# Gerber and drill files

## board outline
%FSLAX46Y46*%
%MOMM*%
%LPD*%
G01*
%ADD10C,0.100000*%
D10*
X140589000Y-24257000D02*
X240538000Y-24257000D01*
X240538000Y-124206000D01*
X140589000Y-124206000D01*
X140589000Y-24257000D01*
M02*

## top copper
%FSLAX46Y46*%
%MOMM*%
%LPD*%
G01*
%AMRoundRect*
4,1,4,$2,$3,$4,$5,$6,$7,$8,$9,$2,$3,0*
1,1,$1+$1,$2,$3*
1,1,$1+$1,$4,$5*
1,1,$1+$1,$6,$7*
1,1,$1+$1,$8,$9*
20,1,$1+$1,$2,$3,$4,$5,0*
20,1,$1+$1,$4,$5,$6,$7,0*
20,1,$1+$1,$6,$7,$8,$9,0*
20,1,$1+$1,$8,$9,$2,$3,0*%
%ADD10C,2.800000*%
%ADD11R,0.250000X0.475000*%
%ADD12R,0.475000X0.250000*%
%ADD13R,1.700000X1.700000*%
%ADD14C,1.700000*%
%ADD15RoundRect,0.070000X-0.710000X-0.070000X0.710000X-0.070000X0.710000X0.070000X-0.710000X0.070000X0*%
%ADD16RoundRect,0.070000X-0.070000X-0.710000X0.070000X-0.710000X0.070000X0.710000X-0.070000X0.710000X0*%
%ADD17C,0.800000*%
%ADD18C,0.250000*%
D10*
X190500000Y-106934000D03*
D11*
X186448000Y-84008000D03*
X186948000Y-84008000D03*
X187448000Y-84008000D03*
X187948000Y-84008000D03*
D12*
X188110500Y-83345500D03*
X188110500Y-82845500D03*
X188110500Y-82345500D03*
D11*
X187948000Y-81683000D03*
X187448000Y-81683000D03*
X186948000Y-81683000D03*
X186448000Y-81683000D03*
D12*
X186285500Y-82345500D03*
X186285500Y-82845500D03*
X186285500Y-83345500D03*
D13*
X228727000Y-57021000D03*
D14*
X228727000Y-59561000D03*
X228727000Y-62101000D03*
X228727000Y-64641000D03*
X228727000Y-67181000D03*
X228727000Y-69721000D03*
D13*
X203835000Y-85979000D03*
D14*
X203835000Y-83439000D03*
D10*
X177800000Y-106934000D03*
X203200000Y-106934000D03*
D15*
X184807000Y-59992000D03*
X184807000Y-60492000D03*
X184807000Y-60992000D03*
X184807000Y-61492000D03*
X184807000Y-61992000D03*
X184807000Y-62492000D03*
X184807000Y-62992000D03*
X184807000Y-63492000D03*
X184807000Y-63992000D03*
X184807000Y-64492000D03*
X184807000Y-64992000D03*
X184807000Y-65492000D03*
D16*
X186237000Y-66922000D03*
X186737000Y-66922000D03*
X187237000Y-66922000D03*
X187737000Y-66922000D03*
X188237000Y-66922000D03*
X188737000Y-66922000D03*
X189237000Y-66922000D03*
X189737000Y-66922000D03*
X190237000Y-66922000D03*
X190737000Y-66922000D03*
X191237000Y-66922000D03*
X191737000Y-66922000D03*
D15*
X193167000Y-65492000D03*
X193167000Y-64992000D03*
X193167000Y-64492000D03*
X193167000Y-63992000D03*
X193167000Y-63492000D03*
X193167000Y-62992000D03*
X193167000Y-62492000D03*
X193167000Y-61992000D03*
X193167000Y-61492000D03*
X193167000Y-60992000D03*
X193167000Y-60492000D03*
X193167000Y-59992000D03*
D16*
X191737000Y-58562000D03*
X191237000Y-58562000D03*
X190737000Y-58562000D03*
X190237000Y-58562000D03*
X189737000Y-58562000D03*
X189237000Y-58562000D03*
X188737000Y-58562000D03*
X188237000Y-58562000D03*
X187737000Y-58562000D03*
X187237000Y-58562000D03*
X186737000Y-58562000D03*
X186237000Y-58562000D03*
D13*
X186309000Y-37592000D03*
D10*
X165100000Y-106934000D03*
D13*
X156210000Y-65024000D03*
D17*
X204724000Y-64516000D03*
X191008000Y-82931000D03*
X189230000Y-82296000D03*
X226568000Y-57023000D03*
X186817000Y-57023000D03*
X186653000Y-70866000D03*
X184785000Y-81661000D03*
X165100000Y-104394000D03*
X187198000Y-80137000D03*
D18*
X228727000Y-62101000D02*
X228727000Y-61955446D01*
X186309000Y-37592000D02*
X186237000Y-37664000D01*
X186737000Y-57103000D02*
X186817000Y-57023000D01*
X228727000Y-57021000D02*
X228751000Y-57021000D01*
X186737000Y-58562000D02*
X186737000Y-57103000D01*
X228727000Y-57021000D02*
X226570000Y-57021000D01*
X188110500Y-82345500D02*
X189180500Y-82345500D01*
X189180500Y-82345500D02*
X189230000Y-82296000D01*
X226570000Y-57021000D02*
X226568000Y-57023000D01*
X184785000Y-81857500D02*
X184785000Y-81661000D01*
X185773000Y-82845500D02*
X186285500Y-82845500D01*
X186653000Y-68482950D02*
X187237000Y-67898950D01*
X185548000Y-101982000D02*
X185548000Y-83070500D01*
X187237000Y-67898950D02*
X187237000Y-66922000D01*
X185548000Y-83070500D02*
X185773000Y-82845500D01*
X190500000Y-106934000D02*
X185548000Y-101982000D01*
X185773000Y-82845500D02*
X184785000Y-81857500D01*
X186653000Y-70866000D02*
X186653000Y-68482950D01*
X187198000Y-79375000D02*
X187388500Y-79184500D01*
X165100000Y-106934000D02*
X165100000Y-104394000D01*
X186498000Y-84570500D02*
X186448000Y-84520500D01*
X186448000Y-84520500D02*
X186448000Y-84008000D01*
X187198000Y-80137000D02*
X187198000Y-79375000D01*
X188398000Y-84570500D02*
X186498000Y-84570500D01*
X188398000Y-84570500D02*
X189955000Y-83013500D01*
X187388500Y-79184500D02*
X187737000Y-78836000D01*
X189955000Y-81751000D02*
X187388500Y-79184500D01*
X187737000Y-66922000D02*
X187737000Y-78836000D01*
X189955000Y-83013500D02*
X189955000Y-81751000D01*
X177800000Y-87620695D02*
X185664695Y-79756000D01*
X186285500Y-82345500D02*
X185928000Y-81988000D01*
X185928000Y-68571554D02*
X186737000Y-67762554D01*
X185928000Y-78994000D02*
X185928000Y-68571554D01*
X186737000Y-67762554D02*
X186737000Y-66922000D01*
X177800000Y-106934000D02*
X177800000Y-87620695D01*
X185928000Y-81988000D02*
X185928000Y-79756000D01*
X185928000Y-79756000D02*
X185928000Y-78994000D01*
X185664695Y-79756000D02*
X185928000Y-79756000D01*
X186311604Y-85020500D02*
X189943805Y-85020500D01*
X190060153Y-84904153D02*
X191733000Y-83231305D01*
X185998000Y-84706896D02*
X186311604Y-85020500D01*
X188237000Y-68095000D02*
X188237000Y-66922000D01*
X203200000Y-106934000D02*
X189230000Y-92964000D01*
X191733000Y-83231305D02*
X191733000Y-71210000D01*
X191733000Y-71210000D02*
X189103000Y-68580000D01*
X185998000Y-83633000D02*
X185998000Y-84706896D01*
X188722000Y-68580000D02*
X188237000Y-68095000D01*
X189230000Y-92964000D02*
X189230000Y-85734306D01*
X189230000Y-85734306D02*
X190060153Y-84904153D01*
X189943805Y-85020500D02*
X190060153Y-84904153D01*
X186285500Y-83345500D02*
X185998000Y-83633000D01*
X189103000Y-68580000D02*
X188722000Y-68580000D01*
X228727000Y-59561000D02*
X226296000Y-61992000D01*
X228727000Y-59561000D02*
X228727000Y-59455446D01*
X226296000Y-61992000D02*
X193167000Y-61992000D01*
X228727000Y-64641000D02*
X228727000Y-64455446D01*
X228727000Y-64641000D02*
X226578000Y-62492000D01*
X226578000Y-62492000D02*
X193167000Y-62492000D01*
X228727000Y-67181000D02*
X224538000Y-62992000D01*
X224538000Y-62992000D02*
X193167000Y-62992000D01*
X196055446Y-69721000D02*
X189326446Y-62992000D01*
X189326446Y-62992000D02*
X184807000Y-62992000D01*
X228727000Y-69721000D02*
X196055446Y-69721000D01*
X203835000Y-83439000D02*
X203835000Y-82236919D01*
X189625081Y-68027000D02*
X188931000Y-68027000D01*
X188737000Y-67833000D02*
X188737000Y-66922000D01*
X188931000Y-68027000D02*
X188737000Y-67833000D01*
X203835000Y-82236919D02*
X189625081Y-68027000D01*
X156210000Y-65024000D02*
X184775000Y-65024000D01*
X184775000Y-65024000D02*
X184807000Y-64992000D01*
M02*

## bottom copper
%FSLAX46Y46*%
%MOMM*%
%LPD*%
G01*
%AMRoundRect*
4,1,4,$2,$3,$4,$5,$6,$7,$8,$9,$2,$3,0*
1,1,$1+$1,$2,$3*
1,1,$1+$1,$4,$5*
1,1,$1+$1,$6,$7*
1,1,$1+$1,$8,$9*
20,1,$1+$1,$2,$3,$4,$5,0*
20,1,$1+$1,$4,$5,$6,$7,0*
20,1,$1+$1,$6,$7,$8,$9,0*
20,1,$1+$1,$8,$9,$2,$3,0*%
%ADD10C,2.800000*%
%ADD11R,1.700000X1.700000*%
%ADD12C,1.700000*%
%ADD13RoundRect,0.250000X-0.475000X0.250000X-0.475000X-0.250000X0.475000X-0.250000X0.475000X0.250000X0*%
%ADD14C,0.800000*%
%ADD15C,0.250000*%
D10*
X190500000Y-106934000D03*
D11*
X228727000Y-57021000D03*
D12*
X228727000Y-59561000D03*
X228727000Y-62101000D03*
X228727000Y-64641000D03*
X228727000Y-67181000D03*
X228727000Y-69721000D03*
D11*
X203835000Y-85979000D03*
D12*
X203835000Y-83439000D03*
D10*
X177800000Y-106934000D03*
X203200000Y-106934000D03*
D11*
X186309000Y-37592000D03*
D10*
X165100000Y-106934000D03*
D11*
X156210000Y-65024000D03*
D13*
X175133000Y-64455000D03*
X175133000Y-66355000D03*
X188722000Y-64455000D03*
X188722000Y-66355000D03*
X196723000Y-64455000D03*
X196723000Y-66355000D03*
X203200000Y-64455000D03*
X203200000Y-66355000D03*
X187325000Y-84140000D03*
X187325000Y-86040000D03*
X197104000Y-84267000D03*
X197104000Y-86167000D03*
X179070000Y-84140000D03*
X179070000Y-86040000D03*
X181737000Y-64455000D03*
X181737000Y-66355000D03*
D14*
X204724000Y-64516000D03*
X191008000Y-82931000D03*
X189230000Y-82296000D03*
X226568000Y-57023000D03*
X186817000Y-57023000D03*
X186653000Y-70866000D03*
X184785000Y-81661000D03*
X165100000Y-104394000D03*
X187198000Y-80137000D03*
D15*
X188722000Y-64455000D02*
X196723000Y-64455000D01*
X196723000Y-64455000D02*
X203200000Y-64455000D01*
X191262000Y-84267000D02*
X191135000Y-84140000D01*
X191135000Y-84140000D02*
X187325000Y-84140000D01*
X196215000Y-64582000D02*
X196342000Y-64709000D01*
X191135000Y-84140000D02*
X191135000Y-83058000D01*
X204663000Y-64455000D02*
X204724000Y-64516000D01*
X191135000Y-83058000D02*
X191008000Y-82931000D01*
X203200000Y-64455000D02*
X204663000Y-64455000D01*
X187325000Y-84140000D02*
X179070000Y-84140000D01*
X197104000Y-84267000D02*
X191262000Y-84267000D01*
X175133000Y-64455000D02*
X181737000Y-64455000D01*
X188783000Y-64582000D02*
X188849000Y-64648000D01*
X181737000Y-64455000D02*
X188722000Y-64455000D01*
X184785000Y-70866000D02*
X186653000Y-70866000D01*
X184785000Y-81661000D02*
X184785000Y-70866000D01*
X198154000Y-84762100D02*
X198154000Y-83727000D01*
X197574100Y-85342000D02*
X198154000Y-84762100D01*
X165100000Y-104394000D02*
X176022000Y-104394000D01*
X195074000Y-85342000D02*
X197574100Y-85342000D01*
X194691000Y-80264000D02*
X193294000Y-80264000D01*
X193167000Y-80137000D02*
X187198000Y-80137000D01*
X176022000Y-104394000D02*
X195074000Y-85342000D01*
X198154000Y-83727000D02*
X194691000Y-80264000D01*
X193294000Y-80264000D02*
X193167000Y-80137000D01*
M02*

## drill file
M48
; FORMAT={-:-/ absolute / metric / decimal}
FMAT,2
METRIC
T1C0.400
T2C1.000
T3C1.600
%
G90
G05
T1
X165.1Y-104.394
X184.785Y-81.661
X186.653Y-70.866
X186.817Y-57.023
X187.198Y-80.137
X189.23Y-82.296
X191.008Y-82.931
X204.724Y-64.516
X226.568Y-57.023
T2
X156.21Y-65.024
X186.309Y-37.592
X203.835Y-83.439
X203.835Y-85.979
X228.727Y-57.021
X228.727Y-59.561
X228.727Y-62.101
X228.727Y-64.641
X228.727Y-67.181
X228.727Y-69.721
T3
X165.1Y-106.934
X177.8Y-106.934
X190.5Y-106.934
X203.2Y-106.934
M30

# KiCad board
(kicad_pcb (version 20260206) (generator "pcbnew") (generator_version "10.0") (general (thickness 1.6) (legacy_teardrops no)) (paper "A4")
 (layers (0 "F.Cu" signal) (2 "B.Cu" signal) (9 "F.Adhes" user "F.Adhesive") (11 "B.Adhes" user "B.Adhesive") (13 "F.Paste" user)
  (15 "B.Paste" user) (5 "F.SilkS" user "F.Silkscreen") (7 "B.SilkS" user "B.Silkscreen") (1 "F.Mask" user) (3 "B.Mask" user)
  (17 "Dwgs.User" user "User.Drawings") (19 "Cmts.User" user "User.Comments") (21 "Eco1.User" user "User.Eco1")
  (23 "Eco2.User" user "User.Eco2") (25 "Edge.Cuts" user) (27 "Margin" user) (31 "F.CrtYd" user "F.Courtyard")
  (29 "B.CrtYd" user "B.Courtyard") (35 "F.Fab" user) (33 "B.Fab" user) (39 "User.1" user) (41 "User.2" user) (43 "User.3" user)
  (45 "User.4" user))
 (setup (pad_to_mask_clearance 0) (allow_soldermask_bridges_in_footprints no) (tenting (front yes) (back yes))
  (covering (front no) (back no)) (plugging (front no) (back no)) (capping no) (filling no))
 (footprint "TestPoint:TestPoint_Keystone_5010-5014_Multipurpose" (layer "F.Cu") (at 190.5 106.934 90)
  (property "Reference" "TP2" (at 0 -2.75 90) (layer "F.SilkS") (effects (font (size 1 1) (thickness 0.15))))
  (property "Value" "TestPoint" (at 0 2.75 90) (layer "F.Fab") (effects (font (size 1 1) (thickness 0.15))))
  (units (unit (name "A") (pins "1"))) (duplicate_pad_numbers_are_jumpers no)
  (pad "1" thru_hole circle (at 0 0 90) (size 2.8 2.8) (drill 1.6) (layers "*.Cu" "*.Mask") (remove_unused_layers no) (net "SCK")))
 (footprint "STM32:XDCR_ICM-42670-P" (layer "F.Cu") (at 187.198 82.8455 90)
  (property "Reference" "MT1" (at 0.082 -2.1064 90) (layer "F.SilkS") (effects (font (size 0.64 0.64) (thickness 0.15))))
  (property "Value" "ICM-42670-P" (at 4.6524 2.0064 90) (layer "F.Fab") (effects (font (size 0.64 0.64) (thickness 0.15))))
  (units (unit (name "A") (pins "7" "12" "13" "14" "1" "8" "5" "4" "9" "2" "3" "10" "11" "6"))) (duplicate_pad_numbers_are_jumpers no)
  (pad "1" smd rect (at -1.1625 -0.75 90) (size 0.475 0.25) (layers "F.Cu") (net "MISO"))
  (pad "2" smd rect (at -1.1625 -0.25 90) (size 0.475 0.25) (layers "F.Cu") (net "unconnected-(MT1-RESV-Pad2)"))
  (pad "3" smd rect (at -1.1625 0.25 90) (size 0.475 0.25) (layers "F.Cu") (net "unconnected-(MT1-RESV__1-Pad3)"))
  (pad "4" smd rect (at -1.1625 0.75 90) (size 0.475 0.25) (layers "F.Cu") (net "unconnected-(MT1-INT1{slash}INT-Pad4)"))
  (pad "5" smd rect (at -0.5 0.9125 90) (size 0.25 0.475) (layers "F.Cu") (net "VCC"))
  (pad "6" smd rect (at 0 0.9125 90) (size 0.25 0.475) (layers "F.Cu") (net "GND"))
  (pad "7" smd rect (at 0.5 0.9125 90) (size 0.25 0.475) (layers "F.Cu") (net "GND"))
  (pad "8" smd rect (at 1.1625 0.75 90) (size 0.475 0.25) (layers "F.Cu") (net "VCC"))
  (pad "9" smd rect (at 1.1625 0.25 90) (size 0.475 0.25) (layers "F.Cu") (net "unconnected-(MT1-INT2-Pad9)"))
  (pad "10" smd rect (at 1.1625 -0.25 90) (size 0.475 0.25) (layers "F.Cu") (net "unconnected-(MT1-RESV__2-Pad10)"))
  (pad "11" smd rect (at 1.1625 -0.75 90) (size 0.475 0.25) (layers "F.Cu") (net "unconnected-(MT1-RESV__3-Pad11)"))
  (pad "12" smd rect (at 0.5 -0.9125 90) (size 0.25 0.475) (layers "F.Cu") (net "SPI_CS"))
  (pad "13" smd rect (at 0 -0.9125 90) (size 0.25 0.475) (layers "F.Cu") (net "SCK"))
  (pad "14" smd rect (at -0.5 -0.9125 90) (size 0.25 0.475) (layers "F.Cu") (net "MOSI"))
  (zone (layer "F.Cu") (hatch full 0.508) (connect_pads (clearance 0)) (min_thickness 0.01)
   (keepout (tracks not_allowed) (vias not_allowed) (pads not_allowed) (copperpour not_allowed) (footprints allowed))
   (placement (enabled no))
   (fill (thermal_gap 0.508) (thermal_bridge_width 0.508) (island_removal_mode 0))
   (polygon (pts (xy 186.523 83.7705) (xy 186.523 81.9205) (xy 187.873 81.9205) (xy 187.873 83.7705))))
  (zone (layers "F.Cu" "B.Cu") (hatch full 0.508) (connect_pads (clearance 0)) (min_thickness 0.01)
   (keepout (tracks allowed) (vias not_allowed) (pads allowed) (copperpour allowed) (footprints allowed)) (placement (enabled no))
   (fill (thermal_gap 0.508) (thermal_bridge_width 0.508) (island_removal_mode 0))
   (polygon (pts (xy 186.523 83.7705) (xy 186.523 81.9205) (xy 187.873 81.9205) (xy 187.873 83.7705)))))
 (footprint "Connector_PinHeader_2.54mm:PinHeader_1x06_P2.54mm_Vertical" (layer "F.Cu") (at 228.727 57.021)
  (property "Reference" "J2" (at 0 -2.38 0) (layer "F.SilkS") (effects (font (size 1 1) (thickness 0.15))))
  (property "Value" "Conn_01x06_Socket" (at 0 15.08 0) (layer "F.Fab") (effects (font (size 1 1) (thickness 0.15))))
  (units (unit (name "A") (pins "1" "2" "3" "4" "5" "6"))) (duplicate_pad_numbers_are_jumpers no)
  (pad "1" thru_hole rect (at 0 0) (size 1.7 1.7) (drill 1) (layers "*.Cu" "*.Mask") (remove_unused_layers no) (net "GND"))
  (pad "2" thru_hole circle (at 0 2.54) (size 1.7 1.7) (drill 1) (layers "*.Cu" "*.Mask") (remove_unused_layers no) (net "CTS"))
  (pad "3" thru_hole circle (at 0 5.08) (size 1.7 1.7) (drill 1) (layers "*.Cu" "*.Mask") (remove_unused_layers no) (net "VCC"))
  (pad "4" thru_hole circle (at 0 7.62) (size 1.7 1.7) (drill 1) (layers "*.Cu" "*.Mask") (remove_unused_layers no) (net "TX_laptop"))
  (pad "5" thru_hole circle (at 0 10.16) (size 1.7 1.7) (drill 1) (layers "*.Cu" "*.Mask") (remove_unused_layers no) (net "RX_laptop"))
  (pad "6" thru_hole circle (at 0 12.7) (size 1.7 1.7) (drill 1) (layers "*.Cu" "*.Mask") (remove_unused_layers no) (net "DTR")))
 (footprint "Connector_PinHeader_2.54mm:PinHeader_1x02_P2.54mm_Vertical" (layer "F.Cu") (at 203.835 85.979 180)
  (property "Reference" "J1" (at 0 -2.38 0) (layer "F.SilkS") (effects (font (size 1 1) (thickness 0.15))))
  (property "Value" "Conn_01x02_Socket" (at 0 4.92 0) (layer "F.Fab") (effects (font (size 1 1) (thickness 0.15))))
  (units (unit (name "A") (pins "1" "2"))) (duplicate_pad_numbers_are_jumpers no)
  (pad "1" thru_hole rect (at 0 0 180) (size 1.7 1.7) (drill 1) (layers "*.Cu" "*.Mask") (remove_unused_layers no) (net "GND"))
  (pad "2" thru_hole circle (at 0 2.54 180) (size 1.7 1.7) (drill 1) (layers "*.Cu" "*.Mask") (remove_unused_layers no) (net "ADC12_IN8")))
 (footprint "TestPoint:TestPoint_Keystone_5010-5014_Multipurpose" (layer "F.Cu") (at 177.8 106.934 90)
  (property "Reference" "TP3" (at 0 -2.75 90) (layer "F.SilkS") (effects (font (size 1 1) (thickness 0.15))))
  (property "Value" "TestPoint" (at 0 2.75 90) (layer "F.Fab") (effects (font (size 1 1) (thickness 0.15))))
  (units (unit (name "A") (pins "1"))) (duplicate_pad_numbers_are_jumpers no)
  (pad "1" thru_hole circle (at 0 0 90) (size 2.8 2.8) (drill 1.6) (layers "*.Cu" "*.Mask") (remove_unused_layers no) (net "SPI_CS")))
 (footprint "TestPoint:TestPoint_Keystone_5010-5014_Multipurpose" (layer "F.Cu") (at 203.2 106.934 90)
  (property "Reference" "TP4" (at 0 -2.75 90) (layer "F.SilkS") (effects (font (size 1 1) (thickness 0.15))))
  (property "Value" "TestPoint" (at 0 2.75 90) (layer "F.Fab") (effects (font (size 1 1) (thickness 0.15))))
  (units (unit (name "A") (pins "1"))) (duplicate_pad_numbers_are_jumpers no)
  (pad "1" thru_hole circle (at 0 0 90) (size 2.8 2.8) (drill 1.6) (layers "*.Cu" "*.Mask") (remove_unused_layers no) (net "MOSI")))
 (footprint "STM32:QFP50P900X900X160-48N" (layer "F.Cu") (at 188.987 62.742)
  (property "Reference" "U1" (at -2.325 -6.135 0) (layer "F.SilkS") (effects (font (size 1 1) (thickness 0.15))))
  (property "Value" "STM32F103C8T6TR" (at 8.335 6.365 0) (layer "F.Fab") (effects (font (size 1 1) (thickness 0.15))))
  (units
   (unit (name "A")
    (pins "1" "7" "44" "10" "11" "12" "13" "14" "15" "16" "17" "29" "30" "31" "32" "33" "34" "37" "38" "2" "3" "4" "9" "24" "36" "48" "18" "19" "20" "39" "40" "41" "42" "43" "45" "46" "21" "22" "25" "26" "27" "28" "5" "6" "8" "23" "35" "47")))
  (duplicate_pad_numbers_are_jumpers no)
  (pad "1" smd roundrect (at -4.18 -2.75) (size 1.56 0.28) (layers "F.Cu" "F.Mask" "F.Paste") (roundrect_rratio 0.25)
   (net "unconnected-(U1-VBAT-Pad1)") (solder_mask_margin 0.102))
  (pad "2" smd roundrect (at -4.18 -2.25) (size 1.56 0.28) (layers "F.Cu" "F.Mask" "F.Paste") (roundrect_rratio 0.25)
   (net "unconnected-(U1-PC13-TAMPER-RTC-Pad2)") (solder_mask_margin 0.102))
  (pad "3" smd roundrect (at -4.18 -1.75) (size 1.56 0.28) (layers "F.Cu" "F.Mask" "F.Paste") (roundrect_rratio 0.25)
   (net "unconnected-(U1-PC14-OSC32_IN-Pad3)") (solder_mask_margin 0.102))
  (pad "4" smd roundrect (at -4.18 -1.25) (size 1.56 0.28) (layers "F.Cu" "F.Mask" "F.Paste") (roundrect_rratio 0.25)
   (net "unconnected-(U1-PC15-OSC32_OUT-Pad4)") (solder_mask_margin 0.102))
  (pad "5" smd roundrect (at -4.18 -0.75) (size 1.56 0.28) (layers "F.Cu" "F.Mask" "F.Paste") (roundrect_rratio 0.25)
   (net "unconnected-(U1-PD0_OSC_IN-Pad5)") (solder_mask_margin 0.102))
  (pad "6" smd roundrect (at -4.18 -0.25) (size 1.56 0.28) (layers "F.Cu" "F.Mask" "F.Paste") (roundrect_rratio 0.25)
   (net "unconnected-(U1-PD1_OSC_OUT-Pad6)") (solder_mask_margin 0.102))
  (pad "7" smd roundrect (at -4.18 0.25) (size 1.56 0.28) (layers "F.Cu" "F.Mask" "F.Paste") (roundrect_rratio 0.25) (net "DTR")
   (solder_mask_margin 0.102))
  (pad "8" smd roundrect (at -4.18 0.75) (size 1.56 0.28) (layers "F.Cu" "F.Mask" "F.Paste") (roundrect_rratio 0.25) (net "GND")
   (solder_mask_margin 0.102))
  (pad "9" smd roundrect (at -4.18 1.25) (size 1.56 0.28) (layers "F.Cu" "F.Mask" "F.Paste") (roundrect_rratio 0.25) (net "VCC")
   (solder_mask_margin 0.102))
  (pad "10" smd roundrect (at -4.18 1.75) (size 1.56 0.28) (layers "F.Cu" "F.Mask" "F.Paste") (roundrect_rratio 0.25)
   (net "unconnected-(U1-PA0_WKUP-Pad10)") (solder_mask_margin 0.102))
  (pad "11" smd roundrect (at -4.18 2.25) (size 1.56 0.28) (layers "F.Cu" "F.Mask" "F.Paste") (roundrect_rratio 0.25) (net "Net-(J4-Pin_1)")
   (solder_mask_margin 0.102))
  (pad "12" smd roundrect (at -4.18 2.75) (size 1.56 0.28) (layers "F.Cu" "F.Mask" "F.Paste") (roundrect_rratio 0.25)
   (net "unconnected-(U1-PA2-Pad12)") (solder_mask_margin 0.102))
  (pad "13" smd roundrect (at -2.75 4.18) (size 0.28 1.56) (layers "F.Cu" "F.Mask" "F.Paste") (roundrect_rratio 0.25)
   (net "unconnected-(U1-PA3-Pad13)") (solder_mask_margin 0.102))
  (pad "14" smd roundrect (at -2.25 4.18) (size 0.28 1.56) (layers "F.Cu" "F.Mask" "F.Paste") (roundrect_rratio 0.25) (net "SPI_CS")
   (solder_mask_margin 0.102))
  (pad "15" smd roundrect (at -1.75 4.18) (size 0.28 1.56) (layers "F.Cu" "F.Mask" "F.Paste") (roundrect_rratio 0.25) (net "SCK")
   (solder_mask_margin 0.102))
  (pad "16" smd roundrect (at -1.25 4.18) (size 0.28 1.56) (layers "F.Cu" "F.Mask" "F.Paste") (roundrect_rratio 0.25) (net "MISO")
   (solder_mask_margin 0.102))
  (pad "17" smd roundrect (at -0.75 4.18) (size 0.28 1.56) (layers "F.Cu" "F.Mask" "F.Paste") (roundrect_rratio 0.25) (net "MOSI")
   (solder_mask_margin 0.102))
  (pad "18" smd roundrect (at -0.25 4.18) (size 0.28 1.56) (layers "F.Cu" "F.Mask" "F.Paste") (roundrect_rratio 0.25) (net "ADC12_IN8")
   (solder_mask_margin 0.102))
  (pad "19" smd roundrect (at 0.25 4.18) (size 0.28 1.56) (layers "F.Cu" "F.Mask" "F.Paste") (roundrect_rratio 0.25)
   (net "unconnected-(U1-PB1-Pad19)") (solder_mask_margin 0.102))
  (pad "20" smd roundrect (at 0.75 4.18) (size 0.28 1.56) (layers "F.Cu" "F.Mask" "F.Paste") (roundrect_rratio 0.25) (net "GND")
   (solder_mask_margin 0.102))
  (pad "21" smd roundrect (at 1.25 4.18) (size 0.28 1.56) (layers "F.Cu" "F.Mask" "F.Paste") (roundrect_rratio 0.25)
   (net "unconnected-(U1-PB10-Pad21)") (solder_mask_margin 0.102))
  (pad "22" smd roundrect (at 1.75 4.18) (size 0.28 1.56) (layers "F.Cu" "F.Mask" "F.Paste") (roundrect_rratio 0.25)
   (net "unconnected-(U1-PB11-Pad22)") (solder_mask_margin 0.102))
  (pad "23" smd roundrect (at 2.25 4.18) (size 0.28 1.56) (layers "F.Cu" "F.Mask" "F.Paste") (roundrect_rratio 0.25) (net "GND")
   (solder_mask_margin 0.102))
  (pad "24" smd roundrect (at 2.75 4.18) (size 0.28 1.56) (layers "F.Cu" "F.Mask" "F.Paste") (roundrect_rratio 0.25) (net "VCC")
   (solder_mask_margin 0.102))
  (pad "25" smd roundrect (at 4.18 2.75) (size 1.56 0.28) (layers "F.Cu" "F.Mask" "F.Paste") (roundrect_rratio 0.25)
   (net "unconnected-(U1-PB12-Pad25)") (solder_mask_margin 0.102))
  (pad "26" smd roundrect (at 4.18 2.25) (size 1.56 0.28) (layers "F.Cu" "F.Mask" "F.Paste") (roundrect_rratio 0.25)
   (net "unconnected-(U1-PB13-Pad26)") (solder_mask_margin 0.102))
  (pad "27" smd roundrect (at 4.18 1.75) (size 1.56 0.28) (layers "F.Cu" "F.Mask" "F.Paste") (roundrect_rratio 0.25)
   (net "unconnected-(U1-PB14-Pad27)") (solder_mask_margin 0.102))
  (pad "28" smd roundrect (at 4.18 1.25) (size 1.56 0.28) (layers "F.Cu" "F.Mask" "F.Paste") (roundrect_rratio 0.25)
   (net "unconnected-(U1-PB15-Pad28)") (solder_mask_margin 0.102))
  (pad "29" smd roundrect (at 4.18 0.75) (size 1.56 0.28) (layers "F.Cu" "F.Mask" "F.Paste") (roundrect_rratio 0.25)
   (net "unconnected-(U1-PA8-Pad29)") (solder_mask_margin 0.102))
  (pad "30" smd roundrect (at 4.18 0.25) (size 1.56 0.28) (layers "F.Cu" "F.Mask" "F.Paste") (roundrect_rratio 0.25) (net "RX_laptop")
   (solder_mask_margin 0.102))
  (pad "31" smd roundrect (at 4.18 -0.25) (size 1.56 0.28) (layers "F.Cu" "F.Mask" "F.Paste") (roundrect_rratio 0.25) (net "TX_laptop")
   (solder_mask_margin 0.102))
  (pad "32" smd roundrect (at 4.18 -0.75) (size 1.56 0.28) (layers "F.Cu" "F.Mask" "F.Paste") (roundrect_rratio 0.25) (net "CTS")
   (solder_mask_margin 0.102))
  (pad "33" smd roundrect (at 4.18 -1.25) (size 1.56 0.28) (layers "F.Cu" "F.Mask" "F.Paste") (roundrect_rratio 0.25)
   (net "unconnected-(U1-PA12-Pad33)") (solder_mask_margin 0.102))
  (pad "34" smd roundrect (at 4.18 -1.75) (size 1.56 0.28) (layers "F.Cu" "F.Mask" "F.Paste") (roundrect_rratio 0.25)
   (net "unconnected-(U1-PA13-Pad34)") (solder_mask_margin 0.102))
  (pad "35" smd roundrect (at 4.18 -2.25) (size 1.56 0.28) (layers "F.Cu" "F.Mask" "F.Paste") (roundrect_rratio 0.25) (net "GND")
   (solder_mask_margin 0.102))
  (pad "36" smd roundrect (at 4.18 -2.75) (size 1.56 0.28) (layers "F.Cu" "F.Mask" "F.Paste") (roundrect_rratio 0.25) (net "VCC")
   (solder_mask_margin 0.102))
  (pad "37" smd roundrect (at 2.75 -4.18) (size 0.28 1.56) (layers "F.Cu" "F.Mask" "F.Paste") (roundrect_rratio 0.25)
   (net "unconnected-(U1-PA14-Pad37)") (solder_mask_margin 0.102))
  (pad "38" smd roundrect (at 2.25 -4.18) (size 0.28 1.56) (layers "F.Cu" "F.Mask" "F.Paste") (roundrect_rratio 0.25)
   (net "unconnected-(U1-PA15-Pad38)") (solder_mask_margin 0.102))
  (pad "39" smd roundrect (at 1.75 -4.18) (size 0.28 1.56) (layers "F.Cu" "F.Mask" "F.Paste") (roundrect_rratio 0.25)
   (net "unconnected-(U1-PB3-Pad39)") (solder_mask_margin 0.102))
  (pad "40" smd roundrect (at 1.25 -4.18) (size 0.28 1.56) (layers "F.Cu" "F.Mask" "F.Paste") (roundrect_rratio 0.25)
   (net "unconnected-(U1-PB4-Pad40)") (solder_mask_margin 0.102))
  (pad "41" smd roundrect (at 0.75 -4.18) (size 0.28 1.56) (layers "F.Cu" "F.Mask" "F.Paste") (roundrect_rratio 0.25)
   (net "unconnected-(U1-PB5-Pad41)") (solder_mask_margin 0.102))
  (pad "42" smd roundrect (at 0.25 -4.18) (size 0.28 1.56) (layers "F.Cu" "F.Mask" "F.Paste") (roundrect_rratio 0.25)
   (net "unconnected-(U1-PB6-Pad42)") (solder_mask_margin 0.102))
  (pad "43" smd roundrect (at -0.25 -4.18) (size 0.28 1.56) (layers "F.Cu" "F.Mask" "F.Paste") (roundrect_rratio 0.25)
   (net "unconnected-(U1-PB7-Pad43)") (solder_mask_margin 0.102))
  (pad "44" smd roundrect (at -0.75 -4.18) (size 0.28 1.56) (layers "F.Cu" "F.Mask" "F.Paste") (roundrect_rratio 0.25) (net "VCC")
   (solder_mask_margin 0.102))
  (pad "45" smd roundrect (at -1.25 -4.18) (size 0.28 1.56) (layers "F.Cu" "F.Mask" "F.Paste") (roundrect_rratio 0.25)
   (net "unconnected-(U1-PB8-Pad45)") (solder_mask_margin 0.102))
  (pad "46" smd roundrect (at -1.75 -4.18) (size 0.28 1.56) (layers "F.Cu" "F.Mask" "F.Paste") (roundrect_rratio 0.25)
   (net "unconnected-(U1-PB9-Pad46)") (solder_mask_margin 0.102))
  (pad "47" smd roundrect (at -2.25 -4.18) (size 0.28 1.56) (layers "F.Cu" "F.Mask" "F.Paste") (roundrect_rratio 0.25) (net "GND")
   (solder_mask_margin 0.102))
  (pad "48" smd roundrect (at -2.75 -4.18) (size 0.28 1.56) (layers "F.Cu" "F.Mask" "F.Paste") (roundrect_rratio 0.25) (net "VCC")
   (solder_mask_margin 0.102)))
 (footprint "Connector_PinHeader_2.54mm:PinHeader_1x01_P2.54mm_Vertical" (layer "F.Cu") (at 186.309 37.592)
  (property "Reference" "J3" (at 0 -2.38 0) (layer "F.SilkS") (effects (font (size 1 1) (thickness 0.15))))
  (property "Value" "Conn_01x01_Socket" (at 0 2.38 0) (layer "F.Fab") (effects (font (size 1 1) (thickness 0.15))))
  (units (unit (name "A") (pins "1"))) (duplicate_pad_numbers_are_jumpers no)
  (pad "1" thru_hole rect (at 0 0) (size 1.7 1.7) (drill 1) (layers "*.Cu" "*.Mask") (remove_unused_layers no) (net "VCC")))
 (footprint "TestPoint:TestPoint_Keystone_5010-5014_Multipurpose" (layer "F.Cu") (at 165.1 106.934 90)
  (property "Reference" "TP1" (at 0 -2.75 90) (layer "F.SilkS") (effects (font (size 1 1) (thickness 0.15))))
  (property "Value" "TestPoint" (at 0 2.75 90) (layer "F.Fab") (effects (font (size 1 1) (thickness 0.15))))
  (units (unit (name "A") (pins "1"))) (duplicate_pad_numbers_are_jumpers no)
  (pad "1" thru_hole circle (at 0 0 90) (size 2.8 2.8) (drill 1.6) (layers "*.Cu" "*.Mask") (remove_unused_layers no) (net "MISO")))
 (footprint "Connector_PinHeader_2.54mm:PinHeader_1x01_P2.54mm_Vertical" (layer "F.Cu") (at 156.21 65.024)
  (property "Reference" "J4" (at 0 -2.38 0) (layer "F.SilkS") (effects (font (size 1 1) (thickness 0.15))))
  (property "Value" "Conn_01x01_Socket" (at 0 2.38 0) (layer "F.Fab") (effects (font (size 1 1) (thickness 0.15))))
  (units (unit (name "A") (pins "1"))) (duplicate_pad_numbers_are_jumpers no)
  (pad "1" thru_hole rect (at 0 0) (size 1.7 1.7) (drill 1) (layers "*.Cu" "*.Mask") (remove_unused_layers no) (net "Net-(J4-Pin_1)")))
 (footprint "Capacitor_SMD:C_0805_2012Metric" (layer "B.Cu") (at 175.133 65.405 -90)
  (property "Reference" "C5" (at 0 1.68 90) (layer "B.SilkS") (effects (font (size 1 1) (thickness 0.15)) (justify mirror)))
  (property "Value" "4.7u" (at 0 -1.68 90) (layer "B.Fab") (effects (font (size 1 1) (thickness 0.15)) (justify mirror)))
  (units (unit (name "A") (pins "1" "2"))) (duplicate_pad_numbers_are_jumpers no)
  (pad "1" smd roundrect (at -0.95 0 270) (size 1 1.45) (layers "B.Cu" "B.Mask" "B.Paste") (roundrect_rratio 0.25) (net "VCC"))
  (pad "2" smd roundrect (at 0.95 0 270) (size 1 1.45) (layers "B.Cu" "B.Mask" "B.Paste") (roundrect_rratio 0.25) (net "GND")))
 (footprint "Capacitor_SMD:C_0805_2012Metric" (layer "B.Cu") (at 188.722 65.405 -90)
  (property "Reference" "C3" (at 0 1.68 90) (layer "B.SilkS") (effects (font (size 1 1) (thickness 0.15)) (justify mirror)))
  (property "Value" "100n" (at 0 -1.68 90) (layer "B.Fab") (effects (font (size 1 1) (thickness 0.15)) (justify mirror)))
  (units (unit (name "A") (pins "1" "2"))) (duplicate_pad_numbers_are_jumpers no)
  (pad "1" smd roundrect (at -0.95 0 270) (size 1 1.45) (layers "B.Cu" "B.Mask" "B.Paste") (roundrect_rratio 0.25) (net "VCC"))
  (pad "2" smd roundrect (at 0.95 0 270) (size 1 1.45) (layers "B.Cu" "B.Mask" "B.Paste") (roundrect_rratio 0.25) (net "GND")))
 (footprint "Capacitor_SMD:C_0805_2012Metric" (layer "B.Cu") (at 196.723 65.405 -90)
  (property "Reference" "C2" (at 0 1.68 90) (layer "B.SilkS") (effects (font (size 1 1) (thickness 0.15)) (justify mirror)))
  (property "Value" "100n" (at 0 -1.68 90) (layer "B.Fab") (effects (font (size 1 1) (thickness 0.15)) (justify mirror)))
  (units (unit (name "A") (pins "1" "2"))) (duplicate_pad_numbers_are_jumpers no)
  (pad "1" smd roundrect (at -0.95 0 270) (size 1 1.45) (layers "B.Cu" "B.Mask" "B.Paste") (roundrect_rratio 0.25) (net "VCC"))
  (pad "2" smd roundrect (at 0.95 0 270) (size 1 1.45) (layers "B.Cu" "B.Mask" "B.Paste") (roundrect_rratio 0.25) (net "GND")))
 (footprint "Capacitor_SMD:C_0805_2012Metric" (layer "B.Cu") (at 203.2 65.405 -90)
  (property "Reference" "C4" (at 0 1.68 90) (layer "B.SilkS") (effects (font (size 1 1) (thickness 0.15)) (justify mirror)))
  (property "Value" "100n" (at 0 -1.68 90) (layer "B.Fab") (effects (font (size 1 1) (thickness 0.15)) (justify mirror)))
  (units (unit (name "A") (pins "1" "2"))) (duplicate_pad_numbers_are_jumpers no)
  (pad "1" smd roundrect (at -0.95 0 270) (size 1 1.45) (layers "B.Cu" "B.Mask" "B.Paste") (roundrect_rratio 0.25) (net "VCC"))
  (pad "2" smd roundrect (at 0.95 0 270) (size 1 1.45) (layers "B.Cu" "B.Mask" "B.Paste") (roundrect_rratio 0.25) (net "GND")))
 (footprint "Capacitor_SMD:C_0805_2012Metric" (layer "B.Cu") (at 187.325 85.09 -90)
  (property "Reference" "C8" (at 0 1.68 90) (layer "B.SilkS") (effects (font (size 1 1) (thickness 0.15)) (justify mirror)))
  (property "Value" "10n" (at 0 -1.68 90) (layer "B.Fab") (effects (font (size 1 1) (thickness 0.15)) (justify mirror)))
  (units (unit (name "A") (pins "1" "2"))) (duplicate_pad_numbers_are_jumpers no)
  (pad "1" smd roundrect (at -0.95 0 270) (size 1 1.45) (layers "B.Cu" "B.Mask" "B.Paste") (roundrect_rratio 0.25) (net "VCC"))
  (pad "2" smd roundrect (at 0.95 0 270) (size 1 1.45) (layers "B.Cu" "B.Mask" "B.Paste") (roundrect_rratio 0.25) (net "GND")))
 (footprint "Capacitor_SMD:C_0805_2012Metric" (layer "B.Cu") (at 197.104 85.217 -90)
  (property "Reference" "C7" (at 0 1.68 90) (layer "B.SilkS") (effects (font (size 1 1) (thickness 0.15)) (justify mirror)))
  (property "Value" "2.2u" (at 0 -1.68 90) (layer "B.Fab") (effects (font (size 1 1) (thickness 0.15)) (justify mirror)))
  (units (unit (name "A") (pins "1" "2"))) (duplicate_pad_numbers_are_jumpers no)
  (pad "1" smd roundrect (at -0.95 0 270) (size 1 1.45) (layers "B.Cu" "B.Mask" "B.Paste") (roundrect_rratio 0.25) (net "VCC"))
  (pad "2" smd roundrect (at 0.95 0 270) (size 1 1.45) (layers "B.Cu" "B.Mask" "B.Paste") (roundrect_rratio 0.25) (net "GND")))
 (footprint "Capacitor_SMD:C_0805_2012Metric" (layer "B.Cu") (at 179.07 85.09 -90)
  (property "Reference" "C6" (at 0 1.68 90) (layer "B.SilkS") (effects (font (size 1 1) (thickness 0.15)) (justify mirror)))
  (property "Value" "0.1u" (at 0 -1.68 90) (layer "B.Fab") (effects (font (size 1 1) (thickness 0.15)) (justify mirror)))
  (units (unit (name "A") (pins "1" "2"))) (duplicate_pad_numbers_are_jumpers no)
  (pad "1" smd roundrect (at -0.95 0 270) (size 1 1.45) (layers "B.Cu" "B.Mask" "B.Paste") (roundrect_rratio 0.25) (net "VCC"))
  (pad "2" smd roundrect (at 0.95 0 270) (size 1 1.45) (layers "B.Cu" "B.Mask" "B.Paste") (roundrect_rratio 0.25) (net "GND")))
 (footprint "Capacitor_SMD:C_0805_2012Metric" (layer "B.Cu") (at 181.737 65.405 -90)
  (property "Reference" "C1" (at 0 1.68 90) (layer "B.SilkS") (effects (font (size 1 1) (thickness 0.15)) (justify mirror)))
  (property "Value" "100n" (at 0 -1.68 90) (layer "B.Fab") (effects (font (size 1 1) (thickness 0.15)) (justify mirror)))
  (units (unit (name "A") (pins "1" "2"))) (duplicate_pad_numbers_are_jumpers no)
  (pad "1" smd roundrect (at -0.95 0 270) (size 1 1.45) (layers "B.Cu" "B.Mask" "B.Paste") (roundrect_rratio 0.25) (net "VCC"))
  (pad "2" smd roundrect (at 0.95 0 270) (size 1 1.45) (layers "B.Cu" "B.Mask" "B.Paste") (roundrect_rratio 0.25) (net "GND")))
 (gr_rect (start 140.589 24.257) (end 240.538 124.206) (stroke (width 0.1) (type default)) (fill no) (layer "Edge.Cuts"))
 (segment (start 228.727 62.101) (end 228.727 61.955446) (width 0.25) (layer "F.Cu") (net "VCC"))
 (segment (start 186.309 37.592) (end 186.237 37.664) (width 0.25) (layer "F.Cu") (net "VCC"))
 (via (at 204.724 64.516) (size 0.8) (drill 0.4) (layers "F.Cu" "B.Cu") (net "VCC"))
 (via (at 191.008 82.931) (size 0.8) (drill 0.4) (layers "F.Cu" "B.Cu") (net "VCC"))
 (segment (start 188.722 64.455) (end 196.723 64.455) (width 0.25) (layer "B.Cu") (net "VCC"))
 (segment (start 196.723 64.455) (end 203.2 64.455) (width 0.25) (layer "B.Cu") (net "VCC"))
 (segment (start 191.262 84.267) (end 191.135 84.14) (width 0.25) (layer "B.Cu") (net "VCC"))
 (segment (start 191.135 84.14) (end 187.325 84.14) (width 0.25) (layer "B.Cu") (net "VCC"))
 (segment (start 196.215 64.582) (end 196.342 64.709) (width 0.25) (layer "B.Cu") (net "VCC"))
 (segment (start 191.135 84.14) (end 191.135 83.058) (width 0.25) (layer "B.Cu") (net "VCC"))
 (segment (start 204.663 64.455) (end 204.724 64.516) (width 0.25) (layer "B.Cu") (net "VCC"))
 (segment (start 191.135 83.058) (end 191.008 82.931) (width 0.25) (layer "B.Cu") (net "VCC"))
 (segment (start 203.2 64.455) (end 204.663 64.455) (width 0.25) (layer "B.Cu") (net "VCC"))
 (segment (start 187.325 84.14) (end 179.07 84.14) (width 0.25) (layer "B.Cu") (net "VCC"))
 (segment (start 197.104 84.267) (end 191.262 84.267) (width 0.25) (layer "B.Cu") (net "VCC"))
 (segment (start 175.133 64.455) (end 181.737 64.455) (width 0.25) (layer "B.Cu") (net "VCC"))
 (segment (start 188.783 64.582) (end 188.849 64.648) (width 0.25) (layer "B.Cu") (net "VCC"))
 (segment (start 181.737 64.455) (end 188.722 64.455) (width 0.25) (layer "B.Cu") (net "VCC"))
 (segment (start 186.737 57.103) (end 186.817 57.023) (width 0.25) (layer "F.Cu") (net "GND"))
 (segment (start 228.727 57.021) (end 228.751 57.021) (width 0.25) (layer "F.Cu") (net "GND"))
 (segment (start 186.737 58.562) (end 186.737 57.103) (width 0.25) (layer "F.Cu") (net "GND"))
 (segment (start 228.727 57.021) (end 226.57 57.021) (width 0.25) (layer "F.Cu") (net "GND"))
 (segment (start 188.1105 82.3455) (end 189.1805 82.3455) (width 0.25) (layer "F.Cu") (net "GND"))
 (segment (start 189.1805 82.3455) (end 189.23 82.296) (width 0.25) (layer "F.Cu") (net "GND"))
 (segment (start 226.57 57.021) (end 226.568 57.023) (width 0.25) (layer "F.Cu") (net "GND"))
 (via (at 189.23 82.296) (size 0.8) (drill 0.4) (layers "F.Cu" "B.Cu") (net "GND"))
 (via (at 226.568 57.023) (size 0.8) (drill 0.4) (layers "F.Cu" "B.Cu") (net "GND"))
 (via (at 186.817 57.023) (size 0.8) (drill 0.4) (layers "F.Cu" "B.Cu") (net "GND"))
 (segment (start 184.785 81.8575) (end 184.785 81.661) (width 0.25) (layer "F.Cu") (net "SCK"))
 (segment (start 185.773 82.8455) (end 186.2855 82.8455) (width 0.25) (layer "F.Cu") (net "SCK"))
 (segment (start 186.653 68.48295) (end 187.237 67.89895) (width 0.25) (layer "F.Cu") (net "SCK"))
 (segment (start 185.548 101.982) (end 185.548 83.0705) (width 0.25) (layer "F.Cu") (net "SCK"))
 (segment (start 187.237 67.89895) (end 187.237 66.922) (width 0.25) (layer "F.Cu") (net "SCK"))
 (segment (start 185.548 83.0705) (end 185.773 82.8455) (width 0.25) (layer "F.Cu") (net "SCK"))
 (segment (start 190.5 106.934) (end 185.548 101.982) (width 0.25) (layer "F.Cu") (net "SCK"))
 (segment (start 185.773 82.8455) (end 184.785 81.8575) (width 0.25) (layer "F.Cu") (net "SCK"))
 (segment (start 186.653 70.866) (end 186.653 68.48295) (width 0.25) (layer "F.Cu") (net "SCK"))
 (via (at 186.653 70.866) (size 0.8) (drill 0.4) (layers "F.Cu" "B.Cu") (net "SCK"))
 (via (at 184.785 81.661) (size 0.8) (drill 0.4) (layers "F.Cu" "B.Cu") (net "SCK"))
 (segment (start 184.785 70.866) (end 186.653 70.866) (width 0.25) (layer "B.Cu") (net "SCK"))
 (segment (start 184.785 81.661) (end 184.785 70.866) (width 0.25) (layer "B.Cu") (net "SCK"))
 (segment (start 187.198 79.375) (end 187.3885 79.1845) (width 0.25) (layer "F.Cu") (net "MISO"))
 (segment (start 165.1 106.934) (end 165.1 104.394) (width 0.25) (layer "F.Cu") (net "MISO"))
 (segment (start 186.498 84.5705) (end 186.448 84.5205) (width 0.25) (layer "F.Cu") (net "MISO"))
 (segment (start 186.448 84.5205) (end 186.448 84.008) (width 0.25) (layer "F.Cu") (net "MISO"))
 (segment (start 187.198 80.137) (end 187.198 79.375) (width 0.25) (layer "F.Cu") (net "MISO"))
 (segment (start 188.398 84.5705) (end 186.498 84.5705) (width 0.25) (layer "F.Cu") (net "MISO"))
 (segment (start 188.398 84.5705) (end 189.955 83.0135) (width 0.25) (layer "F.Cu") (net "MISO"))
 (segment (start 187.3885 79.1845) (end 187.737 78.836) (width 0.25) (layer "F.Cu") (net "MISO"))
 (segment (start 189.955 81.751) (end 187.3885 79.1845) (width 0.25) (layer "F.Cu") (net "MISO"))
 (segment (start 187.737 66.922) (end 187.737 78.836) (width 0.25) (layer "F.Cu") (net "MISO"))
 (segment (start 189.955 83.0135) (end 189.955 81.751) (width 0.25) (layer "F.Cu") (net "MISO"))
 (via (at 165.1 104.394) (size 0.8) (drill 0.4) (layers "F.Cu" "B.Cu") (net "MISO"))
 (via (at 187.198 80.137) (size 0.8) (drill 0.4) (layers "F.Cu" "B.Cu") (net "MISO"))
 (segment (start 198.154 84.7621) (end 198.154 83.727) (width 0.25) (layer "B.Cu") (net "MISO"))
 (segment (start 197.5741 85.342) (end 198.154 84.7621) (width 0.25) (layer "B.Cu") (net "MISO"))
 (segment (start 165.1 104.394) (end 176.022 104.394) (width 0.25) (layer "B.Cu") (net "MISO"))
 (segment (start 195.074 85.342) (end 197.5741 85.342) (width 0.25) (layer "B.Cu") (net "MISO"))
 (segment (start 194.691 80.264) (end 193.294 80.264) (width 0.25) (layer "B.Cu") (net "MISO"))
 (segment (start 193.167 80.137) (end 187.198 80.137) (width 0.25) (layer "B.Cu") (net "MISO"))
 (segment (start 176.022 104.394) (end 195.074 85.342) (width 0.25) (layer "B.Cu") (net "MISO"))
 (segment (start 198.154 83.727) (end 194.691 80.264) (width 0.25) (layer "B.Cu") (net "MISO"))
 (segment (start 193.294 80.264) (end 193.167 80.137) (width 0.25) (layer "B.Cu") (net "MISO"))
 (segment (start 177.8 87.620695) (end 185.664695 79.756) (width 0.25) (layer "F.Cu") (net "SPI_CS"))
 (segment (start 186.2855 82.3455) (end 185.928 81.988) (width 0.25) (layer "F.Cu") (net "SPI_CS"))
 (segment (start 185.928 68.571554) (end 186.737 67.762554) (width 0.25) (layer "F.Cu") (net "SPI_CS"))
 (segment (start 185.928 78.994) (end 185.928 68.571554) (width 0.25) (layer "F.Cu") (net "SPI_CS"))
 (segment (start 186.737 67.762554) (end 186.737 66.922) (width 0.25) (layer "F.Cu") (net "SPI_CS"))
 (segment (start 177.8 106.934) (end 177.8 87.620695) (width 0.25) (layer "F.Cu") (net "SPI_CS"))
 (segment (start 185.928 81.988) (end 185.928 79.756) (width 0.25) (layer "F.Cu") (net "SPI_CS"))
 (segment (start 185.928 79.756) (end 185.928 78.994) (width 0.25) (layer "F.Cu") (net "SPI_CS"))
 (segment (start 185.664695 79.756) (end 185.928 79.756) (width 0.25) (layer "F.Cu") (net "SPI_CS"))
 (segment (start 186.311604 85.0205) (end 189.943805 85.0205) (width 0.25) (layer "F.Cu") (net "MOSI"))
 (segment (start 190.060153 84.904153) (end 191.733 83.231305) (width 0.25) (layer "F.Cu") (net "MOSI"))
 (segment (start 185.998 84.706896) (end 186.311604 85.0205) (width 0.25) (layer "F.Cu") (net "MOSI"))
 (segment (start 188.237 68.095) (end 188.237 66.922) (width 0.25) (layer "F.Cu") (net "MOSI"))
 (segment (start 203.2 106.934) (end 189.23 92.964) (width 0.25) (layer "F.Cu") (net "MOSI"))
 (segment (start 191.733 83.231305) (end 191.733 71.21) (width 0.25) (layer "F.Cu") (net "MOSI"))
 (segment (start 191.733 71.21) (end 189.103 68.58) (width 0.25) (layer "F.Cu") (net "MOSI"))
 (segment (start 185.998 83.633) (end 185.998 84.706896) (width 0.25) (layer "F.Cu") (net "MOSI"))
 (segment (start 188.722 68.58) (end 188.237 68.095) (width 0.25) (layer "F.Cu") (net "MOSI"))
 (segment (start 189.23 92.964) (end 189.23 85.734306) (width 0.25) (layer "F.Cu") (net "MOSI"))
 (segment (start 189.23 85.734306) (end 190.060153 84.904153) (width 0.25) (layer "F.Cu") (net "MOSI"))
 (segment (start 189.943805 85.0205) (end 190.060153 84.904153) (width 0.25) (layer "F.Cu") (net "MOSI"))
 (segment (start 186.2855 83.3455) (end 185.998 83.633) (width 0.25) (layer "F.Cu") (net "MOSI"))
 (segment (start 189.103 68.58) (end 188.722 68.58) (width 0.25) (layer "F.Cu") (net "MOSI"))
 (segment (start 228.727 59.561) (end 226.296 61.992) (width 0.25) (layer "F.Cu") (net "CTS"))
 (segment (start 228.727 59.561) (end 228.727 59.455446) (width 0.25) (layer "F.Cu") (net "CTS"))
 (segment (start 226.296 61.992) (end 193.167 61.992) (width 0.25) (layer "F.Cu") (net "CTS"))
 (segment (start 228.727 64.641) (end 228.727 64.455446) (width 0.25) (layer "F.Cu") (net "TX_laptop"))
 (segment (start 228.727 64.641) (end 226.578 62.492) (width 0.25) (layer "F.Cu") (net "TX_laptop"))
 (segment (start 226.578 62.492) (end 193.167 62.492) (width 0.25) (layer "F.Cu") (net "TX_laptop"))
 (segment (start 228.727 67.181) (end 224.538 62.992) (width 0.25) (layer "F.Cu") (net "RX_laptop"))
 (segment (start 224.538 62.992) (end 193.167 62.992) (width 0.25) (layer "F.Cu") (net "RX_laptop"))
 (segment (start 196.055446 69.721) (end 189.326446 62.992) (width 0.25) (layer "F.Cu") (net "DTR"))
 (segment (start 189.326446 62.992) (end 184.807 62.992) (width 0.25) (layer "F.Cu") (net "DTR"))
 (segment (start 228.727 69.721) (end 196.055446 69.721) (width 0.25) (layer "F.Cu") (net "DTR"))
 (segment (start 203.835 83.439) (end 203.835 82.236919) (width 0.25) (layer "F.Cu") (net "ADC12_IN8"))
 (segment (start 189.625081 68.027) (end 188.931 68.027) (width 0.25) (layer "F.Cu") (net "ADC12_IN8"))
 (segment (start 188.737 67.833) (end 188.737 66.922) (width 0.25) (layer "F.Cu") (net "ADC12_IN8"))
 (segment (start 188.931 68.027) (end 188.737 67.833) (width 0.25) (layer "F.Cu") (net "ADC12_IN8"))
 (segment (start 203.835 82.236919) (end 189.625081 68.027) (width 0.25) (layer "F.Cu") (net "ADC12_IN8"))
 (segment (start 156.21 65.024) (end 184.775 65.024) (width 0.25) (layer "F.Cu") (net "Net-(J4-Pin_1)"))
 (segment (start 184.775 65.024) (end 184.807 64.992) (width 0.25) (layer "F.Cu") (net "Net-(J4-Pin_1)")))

